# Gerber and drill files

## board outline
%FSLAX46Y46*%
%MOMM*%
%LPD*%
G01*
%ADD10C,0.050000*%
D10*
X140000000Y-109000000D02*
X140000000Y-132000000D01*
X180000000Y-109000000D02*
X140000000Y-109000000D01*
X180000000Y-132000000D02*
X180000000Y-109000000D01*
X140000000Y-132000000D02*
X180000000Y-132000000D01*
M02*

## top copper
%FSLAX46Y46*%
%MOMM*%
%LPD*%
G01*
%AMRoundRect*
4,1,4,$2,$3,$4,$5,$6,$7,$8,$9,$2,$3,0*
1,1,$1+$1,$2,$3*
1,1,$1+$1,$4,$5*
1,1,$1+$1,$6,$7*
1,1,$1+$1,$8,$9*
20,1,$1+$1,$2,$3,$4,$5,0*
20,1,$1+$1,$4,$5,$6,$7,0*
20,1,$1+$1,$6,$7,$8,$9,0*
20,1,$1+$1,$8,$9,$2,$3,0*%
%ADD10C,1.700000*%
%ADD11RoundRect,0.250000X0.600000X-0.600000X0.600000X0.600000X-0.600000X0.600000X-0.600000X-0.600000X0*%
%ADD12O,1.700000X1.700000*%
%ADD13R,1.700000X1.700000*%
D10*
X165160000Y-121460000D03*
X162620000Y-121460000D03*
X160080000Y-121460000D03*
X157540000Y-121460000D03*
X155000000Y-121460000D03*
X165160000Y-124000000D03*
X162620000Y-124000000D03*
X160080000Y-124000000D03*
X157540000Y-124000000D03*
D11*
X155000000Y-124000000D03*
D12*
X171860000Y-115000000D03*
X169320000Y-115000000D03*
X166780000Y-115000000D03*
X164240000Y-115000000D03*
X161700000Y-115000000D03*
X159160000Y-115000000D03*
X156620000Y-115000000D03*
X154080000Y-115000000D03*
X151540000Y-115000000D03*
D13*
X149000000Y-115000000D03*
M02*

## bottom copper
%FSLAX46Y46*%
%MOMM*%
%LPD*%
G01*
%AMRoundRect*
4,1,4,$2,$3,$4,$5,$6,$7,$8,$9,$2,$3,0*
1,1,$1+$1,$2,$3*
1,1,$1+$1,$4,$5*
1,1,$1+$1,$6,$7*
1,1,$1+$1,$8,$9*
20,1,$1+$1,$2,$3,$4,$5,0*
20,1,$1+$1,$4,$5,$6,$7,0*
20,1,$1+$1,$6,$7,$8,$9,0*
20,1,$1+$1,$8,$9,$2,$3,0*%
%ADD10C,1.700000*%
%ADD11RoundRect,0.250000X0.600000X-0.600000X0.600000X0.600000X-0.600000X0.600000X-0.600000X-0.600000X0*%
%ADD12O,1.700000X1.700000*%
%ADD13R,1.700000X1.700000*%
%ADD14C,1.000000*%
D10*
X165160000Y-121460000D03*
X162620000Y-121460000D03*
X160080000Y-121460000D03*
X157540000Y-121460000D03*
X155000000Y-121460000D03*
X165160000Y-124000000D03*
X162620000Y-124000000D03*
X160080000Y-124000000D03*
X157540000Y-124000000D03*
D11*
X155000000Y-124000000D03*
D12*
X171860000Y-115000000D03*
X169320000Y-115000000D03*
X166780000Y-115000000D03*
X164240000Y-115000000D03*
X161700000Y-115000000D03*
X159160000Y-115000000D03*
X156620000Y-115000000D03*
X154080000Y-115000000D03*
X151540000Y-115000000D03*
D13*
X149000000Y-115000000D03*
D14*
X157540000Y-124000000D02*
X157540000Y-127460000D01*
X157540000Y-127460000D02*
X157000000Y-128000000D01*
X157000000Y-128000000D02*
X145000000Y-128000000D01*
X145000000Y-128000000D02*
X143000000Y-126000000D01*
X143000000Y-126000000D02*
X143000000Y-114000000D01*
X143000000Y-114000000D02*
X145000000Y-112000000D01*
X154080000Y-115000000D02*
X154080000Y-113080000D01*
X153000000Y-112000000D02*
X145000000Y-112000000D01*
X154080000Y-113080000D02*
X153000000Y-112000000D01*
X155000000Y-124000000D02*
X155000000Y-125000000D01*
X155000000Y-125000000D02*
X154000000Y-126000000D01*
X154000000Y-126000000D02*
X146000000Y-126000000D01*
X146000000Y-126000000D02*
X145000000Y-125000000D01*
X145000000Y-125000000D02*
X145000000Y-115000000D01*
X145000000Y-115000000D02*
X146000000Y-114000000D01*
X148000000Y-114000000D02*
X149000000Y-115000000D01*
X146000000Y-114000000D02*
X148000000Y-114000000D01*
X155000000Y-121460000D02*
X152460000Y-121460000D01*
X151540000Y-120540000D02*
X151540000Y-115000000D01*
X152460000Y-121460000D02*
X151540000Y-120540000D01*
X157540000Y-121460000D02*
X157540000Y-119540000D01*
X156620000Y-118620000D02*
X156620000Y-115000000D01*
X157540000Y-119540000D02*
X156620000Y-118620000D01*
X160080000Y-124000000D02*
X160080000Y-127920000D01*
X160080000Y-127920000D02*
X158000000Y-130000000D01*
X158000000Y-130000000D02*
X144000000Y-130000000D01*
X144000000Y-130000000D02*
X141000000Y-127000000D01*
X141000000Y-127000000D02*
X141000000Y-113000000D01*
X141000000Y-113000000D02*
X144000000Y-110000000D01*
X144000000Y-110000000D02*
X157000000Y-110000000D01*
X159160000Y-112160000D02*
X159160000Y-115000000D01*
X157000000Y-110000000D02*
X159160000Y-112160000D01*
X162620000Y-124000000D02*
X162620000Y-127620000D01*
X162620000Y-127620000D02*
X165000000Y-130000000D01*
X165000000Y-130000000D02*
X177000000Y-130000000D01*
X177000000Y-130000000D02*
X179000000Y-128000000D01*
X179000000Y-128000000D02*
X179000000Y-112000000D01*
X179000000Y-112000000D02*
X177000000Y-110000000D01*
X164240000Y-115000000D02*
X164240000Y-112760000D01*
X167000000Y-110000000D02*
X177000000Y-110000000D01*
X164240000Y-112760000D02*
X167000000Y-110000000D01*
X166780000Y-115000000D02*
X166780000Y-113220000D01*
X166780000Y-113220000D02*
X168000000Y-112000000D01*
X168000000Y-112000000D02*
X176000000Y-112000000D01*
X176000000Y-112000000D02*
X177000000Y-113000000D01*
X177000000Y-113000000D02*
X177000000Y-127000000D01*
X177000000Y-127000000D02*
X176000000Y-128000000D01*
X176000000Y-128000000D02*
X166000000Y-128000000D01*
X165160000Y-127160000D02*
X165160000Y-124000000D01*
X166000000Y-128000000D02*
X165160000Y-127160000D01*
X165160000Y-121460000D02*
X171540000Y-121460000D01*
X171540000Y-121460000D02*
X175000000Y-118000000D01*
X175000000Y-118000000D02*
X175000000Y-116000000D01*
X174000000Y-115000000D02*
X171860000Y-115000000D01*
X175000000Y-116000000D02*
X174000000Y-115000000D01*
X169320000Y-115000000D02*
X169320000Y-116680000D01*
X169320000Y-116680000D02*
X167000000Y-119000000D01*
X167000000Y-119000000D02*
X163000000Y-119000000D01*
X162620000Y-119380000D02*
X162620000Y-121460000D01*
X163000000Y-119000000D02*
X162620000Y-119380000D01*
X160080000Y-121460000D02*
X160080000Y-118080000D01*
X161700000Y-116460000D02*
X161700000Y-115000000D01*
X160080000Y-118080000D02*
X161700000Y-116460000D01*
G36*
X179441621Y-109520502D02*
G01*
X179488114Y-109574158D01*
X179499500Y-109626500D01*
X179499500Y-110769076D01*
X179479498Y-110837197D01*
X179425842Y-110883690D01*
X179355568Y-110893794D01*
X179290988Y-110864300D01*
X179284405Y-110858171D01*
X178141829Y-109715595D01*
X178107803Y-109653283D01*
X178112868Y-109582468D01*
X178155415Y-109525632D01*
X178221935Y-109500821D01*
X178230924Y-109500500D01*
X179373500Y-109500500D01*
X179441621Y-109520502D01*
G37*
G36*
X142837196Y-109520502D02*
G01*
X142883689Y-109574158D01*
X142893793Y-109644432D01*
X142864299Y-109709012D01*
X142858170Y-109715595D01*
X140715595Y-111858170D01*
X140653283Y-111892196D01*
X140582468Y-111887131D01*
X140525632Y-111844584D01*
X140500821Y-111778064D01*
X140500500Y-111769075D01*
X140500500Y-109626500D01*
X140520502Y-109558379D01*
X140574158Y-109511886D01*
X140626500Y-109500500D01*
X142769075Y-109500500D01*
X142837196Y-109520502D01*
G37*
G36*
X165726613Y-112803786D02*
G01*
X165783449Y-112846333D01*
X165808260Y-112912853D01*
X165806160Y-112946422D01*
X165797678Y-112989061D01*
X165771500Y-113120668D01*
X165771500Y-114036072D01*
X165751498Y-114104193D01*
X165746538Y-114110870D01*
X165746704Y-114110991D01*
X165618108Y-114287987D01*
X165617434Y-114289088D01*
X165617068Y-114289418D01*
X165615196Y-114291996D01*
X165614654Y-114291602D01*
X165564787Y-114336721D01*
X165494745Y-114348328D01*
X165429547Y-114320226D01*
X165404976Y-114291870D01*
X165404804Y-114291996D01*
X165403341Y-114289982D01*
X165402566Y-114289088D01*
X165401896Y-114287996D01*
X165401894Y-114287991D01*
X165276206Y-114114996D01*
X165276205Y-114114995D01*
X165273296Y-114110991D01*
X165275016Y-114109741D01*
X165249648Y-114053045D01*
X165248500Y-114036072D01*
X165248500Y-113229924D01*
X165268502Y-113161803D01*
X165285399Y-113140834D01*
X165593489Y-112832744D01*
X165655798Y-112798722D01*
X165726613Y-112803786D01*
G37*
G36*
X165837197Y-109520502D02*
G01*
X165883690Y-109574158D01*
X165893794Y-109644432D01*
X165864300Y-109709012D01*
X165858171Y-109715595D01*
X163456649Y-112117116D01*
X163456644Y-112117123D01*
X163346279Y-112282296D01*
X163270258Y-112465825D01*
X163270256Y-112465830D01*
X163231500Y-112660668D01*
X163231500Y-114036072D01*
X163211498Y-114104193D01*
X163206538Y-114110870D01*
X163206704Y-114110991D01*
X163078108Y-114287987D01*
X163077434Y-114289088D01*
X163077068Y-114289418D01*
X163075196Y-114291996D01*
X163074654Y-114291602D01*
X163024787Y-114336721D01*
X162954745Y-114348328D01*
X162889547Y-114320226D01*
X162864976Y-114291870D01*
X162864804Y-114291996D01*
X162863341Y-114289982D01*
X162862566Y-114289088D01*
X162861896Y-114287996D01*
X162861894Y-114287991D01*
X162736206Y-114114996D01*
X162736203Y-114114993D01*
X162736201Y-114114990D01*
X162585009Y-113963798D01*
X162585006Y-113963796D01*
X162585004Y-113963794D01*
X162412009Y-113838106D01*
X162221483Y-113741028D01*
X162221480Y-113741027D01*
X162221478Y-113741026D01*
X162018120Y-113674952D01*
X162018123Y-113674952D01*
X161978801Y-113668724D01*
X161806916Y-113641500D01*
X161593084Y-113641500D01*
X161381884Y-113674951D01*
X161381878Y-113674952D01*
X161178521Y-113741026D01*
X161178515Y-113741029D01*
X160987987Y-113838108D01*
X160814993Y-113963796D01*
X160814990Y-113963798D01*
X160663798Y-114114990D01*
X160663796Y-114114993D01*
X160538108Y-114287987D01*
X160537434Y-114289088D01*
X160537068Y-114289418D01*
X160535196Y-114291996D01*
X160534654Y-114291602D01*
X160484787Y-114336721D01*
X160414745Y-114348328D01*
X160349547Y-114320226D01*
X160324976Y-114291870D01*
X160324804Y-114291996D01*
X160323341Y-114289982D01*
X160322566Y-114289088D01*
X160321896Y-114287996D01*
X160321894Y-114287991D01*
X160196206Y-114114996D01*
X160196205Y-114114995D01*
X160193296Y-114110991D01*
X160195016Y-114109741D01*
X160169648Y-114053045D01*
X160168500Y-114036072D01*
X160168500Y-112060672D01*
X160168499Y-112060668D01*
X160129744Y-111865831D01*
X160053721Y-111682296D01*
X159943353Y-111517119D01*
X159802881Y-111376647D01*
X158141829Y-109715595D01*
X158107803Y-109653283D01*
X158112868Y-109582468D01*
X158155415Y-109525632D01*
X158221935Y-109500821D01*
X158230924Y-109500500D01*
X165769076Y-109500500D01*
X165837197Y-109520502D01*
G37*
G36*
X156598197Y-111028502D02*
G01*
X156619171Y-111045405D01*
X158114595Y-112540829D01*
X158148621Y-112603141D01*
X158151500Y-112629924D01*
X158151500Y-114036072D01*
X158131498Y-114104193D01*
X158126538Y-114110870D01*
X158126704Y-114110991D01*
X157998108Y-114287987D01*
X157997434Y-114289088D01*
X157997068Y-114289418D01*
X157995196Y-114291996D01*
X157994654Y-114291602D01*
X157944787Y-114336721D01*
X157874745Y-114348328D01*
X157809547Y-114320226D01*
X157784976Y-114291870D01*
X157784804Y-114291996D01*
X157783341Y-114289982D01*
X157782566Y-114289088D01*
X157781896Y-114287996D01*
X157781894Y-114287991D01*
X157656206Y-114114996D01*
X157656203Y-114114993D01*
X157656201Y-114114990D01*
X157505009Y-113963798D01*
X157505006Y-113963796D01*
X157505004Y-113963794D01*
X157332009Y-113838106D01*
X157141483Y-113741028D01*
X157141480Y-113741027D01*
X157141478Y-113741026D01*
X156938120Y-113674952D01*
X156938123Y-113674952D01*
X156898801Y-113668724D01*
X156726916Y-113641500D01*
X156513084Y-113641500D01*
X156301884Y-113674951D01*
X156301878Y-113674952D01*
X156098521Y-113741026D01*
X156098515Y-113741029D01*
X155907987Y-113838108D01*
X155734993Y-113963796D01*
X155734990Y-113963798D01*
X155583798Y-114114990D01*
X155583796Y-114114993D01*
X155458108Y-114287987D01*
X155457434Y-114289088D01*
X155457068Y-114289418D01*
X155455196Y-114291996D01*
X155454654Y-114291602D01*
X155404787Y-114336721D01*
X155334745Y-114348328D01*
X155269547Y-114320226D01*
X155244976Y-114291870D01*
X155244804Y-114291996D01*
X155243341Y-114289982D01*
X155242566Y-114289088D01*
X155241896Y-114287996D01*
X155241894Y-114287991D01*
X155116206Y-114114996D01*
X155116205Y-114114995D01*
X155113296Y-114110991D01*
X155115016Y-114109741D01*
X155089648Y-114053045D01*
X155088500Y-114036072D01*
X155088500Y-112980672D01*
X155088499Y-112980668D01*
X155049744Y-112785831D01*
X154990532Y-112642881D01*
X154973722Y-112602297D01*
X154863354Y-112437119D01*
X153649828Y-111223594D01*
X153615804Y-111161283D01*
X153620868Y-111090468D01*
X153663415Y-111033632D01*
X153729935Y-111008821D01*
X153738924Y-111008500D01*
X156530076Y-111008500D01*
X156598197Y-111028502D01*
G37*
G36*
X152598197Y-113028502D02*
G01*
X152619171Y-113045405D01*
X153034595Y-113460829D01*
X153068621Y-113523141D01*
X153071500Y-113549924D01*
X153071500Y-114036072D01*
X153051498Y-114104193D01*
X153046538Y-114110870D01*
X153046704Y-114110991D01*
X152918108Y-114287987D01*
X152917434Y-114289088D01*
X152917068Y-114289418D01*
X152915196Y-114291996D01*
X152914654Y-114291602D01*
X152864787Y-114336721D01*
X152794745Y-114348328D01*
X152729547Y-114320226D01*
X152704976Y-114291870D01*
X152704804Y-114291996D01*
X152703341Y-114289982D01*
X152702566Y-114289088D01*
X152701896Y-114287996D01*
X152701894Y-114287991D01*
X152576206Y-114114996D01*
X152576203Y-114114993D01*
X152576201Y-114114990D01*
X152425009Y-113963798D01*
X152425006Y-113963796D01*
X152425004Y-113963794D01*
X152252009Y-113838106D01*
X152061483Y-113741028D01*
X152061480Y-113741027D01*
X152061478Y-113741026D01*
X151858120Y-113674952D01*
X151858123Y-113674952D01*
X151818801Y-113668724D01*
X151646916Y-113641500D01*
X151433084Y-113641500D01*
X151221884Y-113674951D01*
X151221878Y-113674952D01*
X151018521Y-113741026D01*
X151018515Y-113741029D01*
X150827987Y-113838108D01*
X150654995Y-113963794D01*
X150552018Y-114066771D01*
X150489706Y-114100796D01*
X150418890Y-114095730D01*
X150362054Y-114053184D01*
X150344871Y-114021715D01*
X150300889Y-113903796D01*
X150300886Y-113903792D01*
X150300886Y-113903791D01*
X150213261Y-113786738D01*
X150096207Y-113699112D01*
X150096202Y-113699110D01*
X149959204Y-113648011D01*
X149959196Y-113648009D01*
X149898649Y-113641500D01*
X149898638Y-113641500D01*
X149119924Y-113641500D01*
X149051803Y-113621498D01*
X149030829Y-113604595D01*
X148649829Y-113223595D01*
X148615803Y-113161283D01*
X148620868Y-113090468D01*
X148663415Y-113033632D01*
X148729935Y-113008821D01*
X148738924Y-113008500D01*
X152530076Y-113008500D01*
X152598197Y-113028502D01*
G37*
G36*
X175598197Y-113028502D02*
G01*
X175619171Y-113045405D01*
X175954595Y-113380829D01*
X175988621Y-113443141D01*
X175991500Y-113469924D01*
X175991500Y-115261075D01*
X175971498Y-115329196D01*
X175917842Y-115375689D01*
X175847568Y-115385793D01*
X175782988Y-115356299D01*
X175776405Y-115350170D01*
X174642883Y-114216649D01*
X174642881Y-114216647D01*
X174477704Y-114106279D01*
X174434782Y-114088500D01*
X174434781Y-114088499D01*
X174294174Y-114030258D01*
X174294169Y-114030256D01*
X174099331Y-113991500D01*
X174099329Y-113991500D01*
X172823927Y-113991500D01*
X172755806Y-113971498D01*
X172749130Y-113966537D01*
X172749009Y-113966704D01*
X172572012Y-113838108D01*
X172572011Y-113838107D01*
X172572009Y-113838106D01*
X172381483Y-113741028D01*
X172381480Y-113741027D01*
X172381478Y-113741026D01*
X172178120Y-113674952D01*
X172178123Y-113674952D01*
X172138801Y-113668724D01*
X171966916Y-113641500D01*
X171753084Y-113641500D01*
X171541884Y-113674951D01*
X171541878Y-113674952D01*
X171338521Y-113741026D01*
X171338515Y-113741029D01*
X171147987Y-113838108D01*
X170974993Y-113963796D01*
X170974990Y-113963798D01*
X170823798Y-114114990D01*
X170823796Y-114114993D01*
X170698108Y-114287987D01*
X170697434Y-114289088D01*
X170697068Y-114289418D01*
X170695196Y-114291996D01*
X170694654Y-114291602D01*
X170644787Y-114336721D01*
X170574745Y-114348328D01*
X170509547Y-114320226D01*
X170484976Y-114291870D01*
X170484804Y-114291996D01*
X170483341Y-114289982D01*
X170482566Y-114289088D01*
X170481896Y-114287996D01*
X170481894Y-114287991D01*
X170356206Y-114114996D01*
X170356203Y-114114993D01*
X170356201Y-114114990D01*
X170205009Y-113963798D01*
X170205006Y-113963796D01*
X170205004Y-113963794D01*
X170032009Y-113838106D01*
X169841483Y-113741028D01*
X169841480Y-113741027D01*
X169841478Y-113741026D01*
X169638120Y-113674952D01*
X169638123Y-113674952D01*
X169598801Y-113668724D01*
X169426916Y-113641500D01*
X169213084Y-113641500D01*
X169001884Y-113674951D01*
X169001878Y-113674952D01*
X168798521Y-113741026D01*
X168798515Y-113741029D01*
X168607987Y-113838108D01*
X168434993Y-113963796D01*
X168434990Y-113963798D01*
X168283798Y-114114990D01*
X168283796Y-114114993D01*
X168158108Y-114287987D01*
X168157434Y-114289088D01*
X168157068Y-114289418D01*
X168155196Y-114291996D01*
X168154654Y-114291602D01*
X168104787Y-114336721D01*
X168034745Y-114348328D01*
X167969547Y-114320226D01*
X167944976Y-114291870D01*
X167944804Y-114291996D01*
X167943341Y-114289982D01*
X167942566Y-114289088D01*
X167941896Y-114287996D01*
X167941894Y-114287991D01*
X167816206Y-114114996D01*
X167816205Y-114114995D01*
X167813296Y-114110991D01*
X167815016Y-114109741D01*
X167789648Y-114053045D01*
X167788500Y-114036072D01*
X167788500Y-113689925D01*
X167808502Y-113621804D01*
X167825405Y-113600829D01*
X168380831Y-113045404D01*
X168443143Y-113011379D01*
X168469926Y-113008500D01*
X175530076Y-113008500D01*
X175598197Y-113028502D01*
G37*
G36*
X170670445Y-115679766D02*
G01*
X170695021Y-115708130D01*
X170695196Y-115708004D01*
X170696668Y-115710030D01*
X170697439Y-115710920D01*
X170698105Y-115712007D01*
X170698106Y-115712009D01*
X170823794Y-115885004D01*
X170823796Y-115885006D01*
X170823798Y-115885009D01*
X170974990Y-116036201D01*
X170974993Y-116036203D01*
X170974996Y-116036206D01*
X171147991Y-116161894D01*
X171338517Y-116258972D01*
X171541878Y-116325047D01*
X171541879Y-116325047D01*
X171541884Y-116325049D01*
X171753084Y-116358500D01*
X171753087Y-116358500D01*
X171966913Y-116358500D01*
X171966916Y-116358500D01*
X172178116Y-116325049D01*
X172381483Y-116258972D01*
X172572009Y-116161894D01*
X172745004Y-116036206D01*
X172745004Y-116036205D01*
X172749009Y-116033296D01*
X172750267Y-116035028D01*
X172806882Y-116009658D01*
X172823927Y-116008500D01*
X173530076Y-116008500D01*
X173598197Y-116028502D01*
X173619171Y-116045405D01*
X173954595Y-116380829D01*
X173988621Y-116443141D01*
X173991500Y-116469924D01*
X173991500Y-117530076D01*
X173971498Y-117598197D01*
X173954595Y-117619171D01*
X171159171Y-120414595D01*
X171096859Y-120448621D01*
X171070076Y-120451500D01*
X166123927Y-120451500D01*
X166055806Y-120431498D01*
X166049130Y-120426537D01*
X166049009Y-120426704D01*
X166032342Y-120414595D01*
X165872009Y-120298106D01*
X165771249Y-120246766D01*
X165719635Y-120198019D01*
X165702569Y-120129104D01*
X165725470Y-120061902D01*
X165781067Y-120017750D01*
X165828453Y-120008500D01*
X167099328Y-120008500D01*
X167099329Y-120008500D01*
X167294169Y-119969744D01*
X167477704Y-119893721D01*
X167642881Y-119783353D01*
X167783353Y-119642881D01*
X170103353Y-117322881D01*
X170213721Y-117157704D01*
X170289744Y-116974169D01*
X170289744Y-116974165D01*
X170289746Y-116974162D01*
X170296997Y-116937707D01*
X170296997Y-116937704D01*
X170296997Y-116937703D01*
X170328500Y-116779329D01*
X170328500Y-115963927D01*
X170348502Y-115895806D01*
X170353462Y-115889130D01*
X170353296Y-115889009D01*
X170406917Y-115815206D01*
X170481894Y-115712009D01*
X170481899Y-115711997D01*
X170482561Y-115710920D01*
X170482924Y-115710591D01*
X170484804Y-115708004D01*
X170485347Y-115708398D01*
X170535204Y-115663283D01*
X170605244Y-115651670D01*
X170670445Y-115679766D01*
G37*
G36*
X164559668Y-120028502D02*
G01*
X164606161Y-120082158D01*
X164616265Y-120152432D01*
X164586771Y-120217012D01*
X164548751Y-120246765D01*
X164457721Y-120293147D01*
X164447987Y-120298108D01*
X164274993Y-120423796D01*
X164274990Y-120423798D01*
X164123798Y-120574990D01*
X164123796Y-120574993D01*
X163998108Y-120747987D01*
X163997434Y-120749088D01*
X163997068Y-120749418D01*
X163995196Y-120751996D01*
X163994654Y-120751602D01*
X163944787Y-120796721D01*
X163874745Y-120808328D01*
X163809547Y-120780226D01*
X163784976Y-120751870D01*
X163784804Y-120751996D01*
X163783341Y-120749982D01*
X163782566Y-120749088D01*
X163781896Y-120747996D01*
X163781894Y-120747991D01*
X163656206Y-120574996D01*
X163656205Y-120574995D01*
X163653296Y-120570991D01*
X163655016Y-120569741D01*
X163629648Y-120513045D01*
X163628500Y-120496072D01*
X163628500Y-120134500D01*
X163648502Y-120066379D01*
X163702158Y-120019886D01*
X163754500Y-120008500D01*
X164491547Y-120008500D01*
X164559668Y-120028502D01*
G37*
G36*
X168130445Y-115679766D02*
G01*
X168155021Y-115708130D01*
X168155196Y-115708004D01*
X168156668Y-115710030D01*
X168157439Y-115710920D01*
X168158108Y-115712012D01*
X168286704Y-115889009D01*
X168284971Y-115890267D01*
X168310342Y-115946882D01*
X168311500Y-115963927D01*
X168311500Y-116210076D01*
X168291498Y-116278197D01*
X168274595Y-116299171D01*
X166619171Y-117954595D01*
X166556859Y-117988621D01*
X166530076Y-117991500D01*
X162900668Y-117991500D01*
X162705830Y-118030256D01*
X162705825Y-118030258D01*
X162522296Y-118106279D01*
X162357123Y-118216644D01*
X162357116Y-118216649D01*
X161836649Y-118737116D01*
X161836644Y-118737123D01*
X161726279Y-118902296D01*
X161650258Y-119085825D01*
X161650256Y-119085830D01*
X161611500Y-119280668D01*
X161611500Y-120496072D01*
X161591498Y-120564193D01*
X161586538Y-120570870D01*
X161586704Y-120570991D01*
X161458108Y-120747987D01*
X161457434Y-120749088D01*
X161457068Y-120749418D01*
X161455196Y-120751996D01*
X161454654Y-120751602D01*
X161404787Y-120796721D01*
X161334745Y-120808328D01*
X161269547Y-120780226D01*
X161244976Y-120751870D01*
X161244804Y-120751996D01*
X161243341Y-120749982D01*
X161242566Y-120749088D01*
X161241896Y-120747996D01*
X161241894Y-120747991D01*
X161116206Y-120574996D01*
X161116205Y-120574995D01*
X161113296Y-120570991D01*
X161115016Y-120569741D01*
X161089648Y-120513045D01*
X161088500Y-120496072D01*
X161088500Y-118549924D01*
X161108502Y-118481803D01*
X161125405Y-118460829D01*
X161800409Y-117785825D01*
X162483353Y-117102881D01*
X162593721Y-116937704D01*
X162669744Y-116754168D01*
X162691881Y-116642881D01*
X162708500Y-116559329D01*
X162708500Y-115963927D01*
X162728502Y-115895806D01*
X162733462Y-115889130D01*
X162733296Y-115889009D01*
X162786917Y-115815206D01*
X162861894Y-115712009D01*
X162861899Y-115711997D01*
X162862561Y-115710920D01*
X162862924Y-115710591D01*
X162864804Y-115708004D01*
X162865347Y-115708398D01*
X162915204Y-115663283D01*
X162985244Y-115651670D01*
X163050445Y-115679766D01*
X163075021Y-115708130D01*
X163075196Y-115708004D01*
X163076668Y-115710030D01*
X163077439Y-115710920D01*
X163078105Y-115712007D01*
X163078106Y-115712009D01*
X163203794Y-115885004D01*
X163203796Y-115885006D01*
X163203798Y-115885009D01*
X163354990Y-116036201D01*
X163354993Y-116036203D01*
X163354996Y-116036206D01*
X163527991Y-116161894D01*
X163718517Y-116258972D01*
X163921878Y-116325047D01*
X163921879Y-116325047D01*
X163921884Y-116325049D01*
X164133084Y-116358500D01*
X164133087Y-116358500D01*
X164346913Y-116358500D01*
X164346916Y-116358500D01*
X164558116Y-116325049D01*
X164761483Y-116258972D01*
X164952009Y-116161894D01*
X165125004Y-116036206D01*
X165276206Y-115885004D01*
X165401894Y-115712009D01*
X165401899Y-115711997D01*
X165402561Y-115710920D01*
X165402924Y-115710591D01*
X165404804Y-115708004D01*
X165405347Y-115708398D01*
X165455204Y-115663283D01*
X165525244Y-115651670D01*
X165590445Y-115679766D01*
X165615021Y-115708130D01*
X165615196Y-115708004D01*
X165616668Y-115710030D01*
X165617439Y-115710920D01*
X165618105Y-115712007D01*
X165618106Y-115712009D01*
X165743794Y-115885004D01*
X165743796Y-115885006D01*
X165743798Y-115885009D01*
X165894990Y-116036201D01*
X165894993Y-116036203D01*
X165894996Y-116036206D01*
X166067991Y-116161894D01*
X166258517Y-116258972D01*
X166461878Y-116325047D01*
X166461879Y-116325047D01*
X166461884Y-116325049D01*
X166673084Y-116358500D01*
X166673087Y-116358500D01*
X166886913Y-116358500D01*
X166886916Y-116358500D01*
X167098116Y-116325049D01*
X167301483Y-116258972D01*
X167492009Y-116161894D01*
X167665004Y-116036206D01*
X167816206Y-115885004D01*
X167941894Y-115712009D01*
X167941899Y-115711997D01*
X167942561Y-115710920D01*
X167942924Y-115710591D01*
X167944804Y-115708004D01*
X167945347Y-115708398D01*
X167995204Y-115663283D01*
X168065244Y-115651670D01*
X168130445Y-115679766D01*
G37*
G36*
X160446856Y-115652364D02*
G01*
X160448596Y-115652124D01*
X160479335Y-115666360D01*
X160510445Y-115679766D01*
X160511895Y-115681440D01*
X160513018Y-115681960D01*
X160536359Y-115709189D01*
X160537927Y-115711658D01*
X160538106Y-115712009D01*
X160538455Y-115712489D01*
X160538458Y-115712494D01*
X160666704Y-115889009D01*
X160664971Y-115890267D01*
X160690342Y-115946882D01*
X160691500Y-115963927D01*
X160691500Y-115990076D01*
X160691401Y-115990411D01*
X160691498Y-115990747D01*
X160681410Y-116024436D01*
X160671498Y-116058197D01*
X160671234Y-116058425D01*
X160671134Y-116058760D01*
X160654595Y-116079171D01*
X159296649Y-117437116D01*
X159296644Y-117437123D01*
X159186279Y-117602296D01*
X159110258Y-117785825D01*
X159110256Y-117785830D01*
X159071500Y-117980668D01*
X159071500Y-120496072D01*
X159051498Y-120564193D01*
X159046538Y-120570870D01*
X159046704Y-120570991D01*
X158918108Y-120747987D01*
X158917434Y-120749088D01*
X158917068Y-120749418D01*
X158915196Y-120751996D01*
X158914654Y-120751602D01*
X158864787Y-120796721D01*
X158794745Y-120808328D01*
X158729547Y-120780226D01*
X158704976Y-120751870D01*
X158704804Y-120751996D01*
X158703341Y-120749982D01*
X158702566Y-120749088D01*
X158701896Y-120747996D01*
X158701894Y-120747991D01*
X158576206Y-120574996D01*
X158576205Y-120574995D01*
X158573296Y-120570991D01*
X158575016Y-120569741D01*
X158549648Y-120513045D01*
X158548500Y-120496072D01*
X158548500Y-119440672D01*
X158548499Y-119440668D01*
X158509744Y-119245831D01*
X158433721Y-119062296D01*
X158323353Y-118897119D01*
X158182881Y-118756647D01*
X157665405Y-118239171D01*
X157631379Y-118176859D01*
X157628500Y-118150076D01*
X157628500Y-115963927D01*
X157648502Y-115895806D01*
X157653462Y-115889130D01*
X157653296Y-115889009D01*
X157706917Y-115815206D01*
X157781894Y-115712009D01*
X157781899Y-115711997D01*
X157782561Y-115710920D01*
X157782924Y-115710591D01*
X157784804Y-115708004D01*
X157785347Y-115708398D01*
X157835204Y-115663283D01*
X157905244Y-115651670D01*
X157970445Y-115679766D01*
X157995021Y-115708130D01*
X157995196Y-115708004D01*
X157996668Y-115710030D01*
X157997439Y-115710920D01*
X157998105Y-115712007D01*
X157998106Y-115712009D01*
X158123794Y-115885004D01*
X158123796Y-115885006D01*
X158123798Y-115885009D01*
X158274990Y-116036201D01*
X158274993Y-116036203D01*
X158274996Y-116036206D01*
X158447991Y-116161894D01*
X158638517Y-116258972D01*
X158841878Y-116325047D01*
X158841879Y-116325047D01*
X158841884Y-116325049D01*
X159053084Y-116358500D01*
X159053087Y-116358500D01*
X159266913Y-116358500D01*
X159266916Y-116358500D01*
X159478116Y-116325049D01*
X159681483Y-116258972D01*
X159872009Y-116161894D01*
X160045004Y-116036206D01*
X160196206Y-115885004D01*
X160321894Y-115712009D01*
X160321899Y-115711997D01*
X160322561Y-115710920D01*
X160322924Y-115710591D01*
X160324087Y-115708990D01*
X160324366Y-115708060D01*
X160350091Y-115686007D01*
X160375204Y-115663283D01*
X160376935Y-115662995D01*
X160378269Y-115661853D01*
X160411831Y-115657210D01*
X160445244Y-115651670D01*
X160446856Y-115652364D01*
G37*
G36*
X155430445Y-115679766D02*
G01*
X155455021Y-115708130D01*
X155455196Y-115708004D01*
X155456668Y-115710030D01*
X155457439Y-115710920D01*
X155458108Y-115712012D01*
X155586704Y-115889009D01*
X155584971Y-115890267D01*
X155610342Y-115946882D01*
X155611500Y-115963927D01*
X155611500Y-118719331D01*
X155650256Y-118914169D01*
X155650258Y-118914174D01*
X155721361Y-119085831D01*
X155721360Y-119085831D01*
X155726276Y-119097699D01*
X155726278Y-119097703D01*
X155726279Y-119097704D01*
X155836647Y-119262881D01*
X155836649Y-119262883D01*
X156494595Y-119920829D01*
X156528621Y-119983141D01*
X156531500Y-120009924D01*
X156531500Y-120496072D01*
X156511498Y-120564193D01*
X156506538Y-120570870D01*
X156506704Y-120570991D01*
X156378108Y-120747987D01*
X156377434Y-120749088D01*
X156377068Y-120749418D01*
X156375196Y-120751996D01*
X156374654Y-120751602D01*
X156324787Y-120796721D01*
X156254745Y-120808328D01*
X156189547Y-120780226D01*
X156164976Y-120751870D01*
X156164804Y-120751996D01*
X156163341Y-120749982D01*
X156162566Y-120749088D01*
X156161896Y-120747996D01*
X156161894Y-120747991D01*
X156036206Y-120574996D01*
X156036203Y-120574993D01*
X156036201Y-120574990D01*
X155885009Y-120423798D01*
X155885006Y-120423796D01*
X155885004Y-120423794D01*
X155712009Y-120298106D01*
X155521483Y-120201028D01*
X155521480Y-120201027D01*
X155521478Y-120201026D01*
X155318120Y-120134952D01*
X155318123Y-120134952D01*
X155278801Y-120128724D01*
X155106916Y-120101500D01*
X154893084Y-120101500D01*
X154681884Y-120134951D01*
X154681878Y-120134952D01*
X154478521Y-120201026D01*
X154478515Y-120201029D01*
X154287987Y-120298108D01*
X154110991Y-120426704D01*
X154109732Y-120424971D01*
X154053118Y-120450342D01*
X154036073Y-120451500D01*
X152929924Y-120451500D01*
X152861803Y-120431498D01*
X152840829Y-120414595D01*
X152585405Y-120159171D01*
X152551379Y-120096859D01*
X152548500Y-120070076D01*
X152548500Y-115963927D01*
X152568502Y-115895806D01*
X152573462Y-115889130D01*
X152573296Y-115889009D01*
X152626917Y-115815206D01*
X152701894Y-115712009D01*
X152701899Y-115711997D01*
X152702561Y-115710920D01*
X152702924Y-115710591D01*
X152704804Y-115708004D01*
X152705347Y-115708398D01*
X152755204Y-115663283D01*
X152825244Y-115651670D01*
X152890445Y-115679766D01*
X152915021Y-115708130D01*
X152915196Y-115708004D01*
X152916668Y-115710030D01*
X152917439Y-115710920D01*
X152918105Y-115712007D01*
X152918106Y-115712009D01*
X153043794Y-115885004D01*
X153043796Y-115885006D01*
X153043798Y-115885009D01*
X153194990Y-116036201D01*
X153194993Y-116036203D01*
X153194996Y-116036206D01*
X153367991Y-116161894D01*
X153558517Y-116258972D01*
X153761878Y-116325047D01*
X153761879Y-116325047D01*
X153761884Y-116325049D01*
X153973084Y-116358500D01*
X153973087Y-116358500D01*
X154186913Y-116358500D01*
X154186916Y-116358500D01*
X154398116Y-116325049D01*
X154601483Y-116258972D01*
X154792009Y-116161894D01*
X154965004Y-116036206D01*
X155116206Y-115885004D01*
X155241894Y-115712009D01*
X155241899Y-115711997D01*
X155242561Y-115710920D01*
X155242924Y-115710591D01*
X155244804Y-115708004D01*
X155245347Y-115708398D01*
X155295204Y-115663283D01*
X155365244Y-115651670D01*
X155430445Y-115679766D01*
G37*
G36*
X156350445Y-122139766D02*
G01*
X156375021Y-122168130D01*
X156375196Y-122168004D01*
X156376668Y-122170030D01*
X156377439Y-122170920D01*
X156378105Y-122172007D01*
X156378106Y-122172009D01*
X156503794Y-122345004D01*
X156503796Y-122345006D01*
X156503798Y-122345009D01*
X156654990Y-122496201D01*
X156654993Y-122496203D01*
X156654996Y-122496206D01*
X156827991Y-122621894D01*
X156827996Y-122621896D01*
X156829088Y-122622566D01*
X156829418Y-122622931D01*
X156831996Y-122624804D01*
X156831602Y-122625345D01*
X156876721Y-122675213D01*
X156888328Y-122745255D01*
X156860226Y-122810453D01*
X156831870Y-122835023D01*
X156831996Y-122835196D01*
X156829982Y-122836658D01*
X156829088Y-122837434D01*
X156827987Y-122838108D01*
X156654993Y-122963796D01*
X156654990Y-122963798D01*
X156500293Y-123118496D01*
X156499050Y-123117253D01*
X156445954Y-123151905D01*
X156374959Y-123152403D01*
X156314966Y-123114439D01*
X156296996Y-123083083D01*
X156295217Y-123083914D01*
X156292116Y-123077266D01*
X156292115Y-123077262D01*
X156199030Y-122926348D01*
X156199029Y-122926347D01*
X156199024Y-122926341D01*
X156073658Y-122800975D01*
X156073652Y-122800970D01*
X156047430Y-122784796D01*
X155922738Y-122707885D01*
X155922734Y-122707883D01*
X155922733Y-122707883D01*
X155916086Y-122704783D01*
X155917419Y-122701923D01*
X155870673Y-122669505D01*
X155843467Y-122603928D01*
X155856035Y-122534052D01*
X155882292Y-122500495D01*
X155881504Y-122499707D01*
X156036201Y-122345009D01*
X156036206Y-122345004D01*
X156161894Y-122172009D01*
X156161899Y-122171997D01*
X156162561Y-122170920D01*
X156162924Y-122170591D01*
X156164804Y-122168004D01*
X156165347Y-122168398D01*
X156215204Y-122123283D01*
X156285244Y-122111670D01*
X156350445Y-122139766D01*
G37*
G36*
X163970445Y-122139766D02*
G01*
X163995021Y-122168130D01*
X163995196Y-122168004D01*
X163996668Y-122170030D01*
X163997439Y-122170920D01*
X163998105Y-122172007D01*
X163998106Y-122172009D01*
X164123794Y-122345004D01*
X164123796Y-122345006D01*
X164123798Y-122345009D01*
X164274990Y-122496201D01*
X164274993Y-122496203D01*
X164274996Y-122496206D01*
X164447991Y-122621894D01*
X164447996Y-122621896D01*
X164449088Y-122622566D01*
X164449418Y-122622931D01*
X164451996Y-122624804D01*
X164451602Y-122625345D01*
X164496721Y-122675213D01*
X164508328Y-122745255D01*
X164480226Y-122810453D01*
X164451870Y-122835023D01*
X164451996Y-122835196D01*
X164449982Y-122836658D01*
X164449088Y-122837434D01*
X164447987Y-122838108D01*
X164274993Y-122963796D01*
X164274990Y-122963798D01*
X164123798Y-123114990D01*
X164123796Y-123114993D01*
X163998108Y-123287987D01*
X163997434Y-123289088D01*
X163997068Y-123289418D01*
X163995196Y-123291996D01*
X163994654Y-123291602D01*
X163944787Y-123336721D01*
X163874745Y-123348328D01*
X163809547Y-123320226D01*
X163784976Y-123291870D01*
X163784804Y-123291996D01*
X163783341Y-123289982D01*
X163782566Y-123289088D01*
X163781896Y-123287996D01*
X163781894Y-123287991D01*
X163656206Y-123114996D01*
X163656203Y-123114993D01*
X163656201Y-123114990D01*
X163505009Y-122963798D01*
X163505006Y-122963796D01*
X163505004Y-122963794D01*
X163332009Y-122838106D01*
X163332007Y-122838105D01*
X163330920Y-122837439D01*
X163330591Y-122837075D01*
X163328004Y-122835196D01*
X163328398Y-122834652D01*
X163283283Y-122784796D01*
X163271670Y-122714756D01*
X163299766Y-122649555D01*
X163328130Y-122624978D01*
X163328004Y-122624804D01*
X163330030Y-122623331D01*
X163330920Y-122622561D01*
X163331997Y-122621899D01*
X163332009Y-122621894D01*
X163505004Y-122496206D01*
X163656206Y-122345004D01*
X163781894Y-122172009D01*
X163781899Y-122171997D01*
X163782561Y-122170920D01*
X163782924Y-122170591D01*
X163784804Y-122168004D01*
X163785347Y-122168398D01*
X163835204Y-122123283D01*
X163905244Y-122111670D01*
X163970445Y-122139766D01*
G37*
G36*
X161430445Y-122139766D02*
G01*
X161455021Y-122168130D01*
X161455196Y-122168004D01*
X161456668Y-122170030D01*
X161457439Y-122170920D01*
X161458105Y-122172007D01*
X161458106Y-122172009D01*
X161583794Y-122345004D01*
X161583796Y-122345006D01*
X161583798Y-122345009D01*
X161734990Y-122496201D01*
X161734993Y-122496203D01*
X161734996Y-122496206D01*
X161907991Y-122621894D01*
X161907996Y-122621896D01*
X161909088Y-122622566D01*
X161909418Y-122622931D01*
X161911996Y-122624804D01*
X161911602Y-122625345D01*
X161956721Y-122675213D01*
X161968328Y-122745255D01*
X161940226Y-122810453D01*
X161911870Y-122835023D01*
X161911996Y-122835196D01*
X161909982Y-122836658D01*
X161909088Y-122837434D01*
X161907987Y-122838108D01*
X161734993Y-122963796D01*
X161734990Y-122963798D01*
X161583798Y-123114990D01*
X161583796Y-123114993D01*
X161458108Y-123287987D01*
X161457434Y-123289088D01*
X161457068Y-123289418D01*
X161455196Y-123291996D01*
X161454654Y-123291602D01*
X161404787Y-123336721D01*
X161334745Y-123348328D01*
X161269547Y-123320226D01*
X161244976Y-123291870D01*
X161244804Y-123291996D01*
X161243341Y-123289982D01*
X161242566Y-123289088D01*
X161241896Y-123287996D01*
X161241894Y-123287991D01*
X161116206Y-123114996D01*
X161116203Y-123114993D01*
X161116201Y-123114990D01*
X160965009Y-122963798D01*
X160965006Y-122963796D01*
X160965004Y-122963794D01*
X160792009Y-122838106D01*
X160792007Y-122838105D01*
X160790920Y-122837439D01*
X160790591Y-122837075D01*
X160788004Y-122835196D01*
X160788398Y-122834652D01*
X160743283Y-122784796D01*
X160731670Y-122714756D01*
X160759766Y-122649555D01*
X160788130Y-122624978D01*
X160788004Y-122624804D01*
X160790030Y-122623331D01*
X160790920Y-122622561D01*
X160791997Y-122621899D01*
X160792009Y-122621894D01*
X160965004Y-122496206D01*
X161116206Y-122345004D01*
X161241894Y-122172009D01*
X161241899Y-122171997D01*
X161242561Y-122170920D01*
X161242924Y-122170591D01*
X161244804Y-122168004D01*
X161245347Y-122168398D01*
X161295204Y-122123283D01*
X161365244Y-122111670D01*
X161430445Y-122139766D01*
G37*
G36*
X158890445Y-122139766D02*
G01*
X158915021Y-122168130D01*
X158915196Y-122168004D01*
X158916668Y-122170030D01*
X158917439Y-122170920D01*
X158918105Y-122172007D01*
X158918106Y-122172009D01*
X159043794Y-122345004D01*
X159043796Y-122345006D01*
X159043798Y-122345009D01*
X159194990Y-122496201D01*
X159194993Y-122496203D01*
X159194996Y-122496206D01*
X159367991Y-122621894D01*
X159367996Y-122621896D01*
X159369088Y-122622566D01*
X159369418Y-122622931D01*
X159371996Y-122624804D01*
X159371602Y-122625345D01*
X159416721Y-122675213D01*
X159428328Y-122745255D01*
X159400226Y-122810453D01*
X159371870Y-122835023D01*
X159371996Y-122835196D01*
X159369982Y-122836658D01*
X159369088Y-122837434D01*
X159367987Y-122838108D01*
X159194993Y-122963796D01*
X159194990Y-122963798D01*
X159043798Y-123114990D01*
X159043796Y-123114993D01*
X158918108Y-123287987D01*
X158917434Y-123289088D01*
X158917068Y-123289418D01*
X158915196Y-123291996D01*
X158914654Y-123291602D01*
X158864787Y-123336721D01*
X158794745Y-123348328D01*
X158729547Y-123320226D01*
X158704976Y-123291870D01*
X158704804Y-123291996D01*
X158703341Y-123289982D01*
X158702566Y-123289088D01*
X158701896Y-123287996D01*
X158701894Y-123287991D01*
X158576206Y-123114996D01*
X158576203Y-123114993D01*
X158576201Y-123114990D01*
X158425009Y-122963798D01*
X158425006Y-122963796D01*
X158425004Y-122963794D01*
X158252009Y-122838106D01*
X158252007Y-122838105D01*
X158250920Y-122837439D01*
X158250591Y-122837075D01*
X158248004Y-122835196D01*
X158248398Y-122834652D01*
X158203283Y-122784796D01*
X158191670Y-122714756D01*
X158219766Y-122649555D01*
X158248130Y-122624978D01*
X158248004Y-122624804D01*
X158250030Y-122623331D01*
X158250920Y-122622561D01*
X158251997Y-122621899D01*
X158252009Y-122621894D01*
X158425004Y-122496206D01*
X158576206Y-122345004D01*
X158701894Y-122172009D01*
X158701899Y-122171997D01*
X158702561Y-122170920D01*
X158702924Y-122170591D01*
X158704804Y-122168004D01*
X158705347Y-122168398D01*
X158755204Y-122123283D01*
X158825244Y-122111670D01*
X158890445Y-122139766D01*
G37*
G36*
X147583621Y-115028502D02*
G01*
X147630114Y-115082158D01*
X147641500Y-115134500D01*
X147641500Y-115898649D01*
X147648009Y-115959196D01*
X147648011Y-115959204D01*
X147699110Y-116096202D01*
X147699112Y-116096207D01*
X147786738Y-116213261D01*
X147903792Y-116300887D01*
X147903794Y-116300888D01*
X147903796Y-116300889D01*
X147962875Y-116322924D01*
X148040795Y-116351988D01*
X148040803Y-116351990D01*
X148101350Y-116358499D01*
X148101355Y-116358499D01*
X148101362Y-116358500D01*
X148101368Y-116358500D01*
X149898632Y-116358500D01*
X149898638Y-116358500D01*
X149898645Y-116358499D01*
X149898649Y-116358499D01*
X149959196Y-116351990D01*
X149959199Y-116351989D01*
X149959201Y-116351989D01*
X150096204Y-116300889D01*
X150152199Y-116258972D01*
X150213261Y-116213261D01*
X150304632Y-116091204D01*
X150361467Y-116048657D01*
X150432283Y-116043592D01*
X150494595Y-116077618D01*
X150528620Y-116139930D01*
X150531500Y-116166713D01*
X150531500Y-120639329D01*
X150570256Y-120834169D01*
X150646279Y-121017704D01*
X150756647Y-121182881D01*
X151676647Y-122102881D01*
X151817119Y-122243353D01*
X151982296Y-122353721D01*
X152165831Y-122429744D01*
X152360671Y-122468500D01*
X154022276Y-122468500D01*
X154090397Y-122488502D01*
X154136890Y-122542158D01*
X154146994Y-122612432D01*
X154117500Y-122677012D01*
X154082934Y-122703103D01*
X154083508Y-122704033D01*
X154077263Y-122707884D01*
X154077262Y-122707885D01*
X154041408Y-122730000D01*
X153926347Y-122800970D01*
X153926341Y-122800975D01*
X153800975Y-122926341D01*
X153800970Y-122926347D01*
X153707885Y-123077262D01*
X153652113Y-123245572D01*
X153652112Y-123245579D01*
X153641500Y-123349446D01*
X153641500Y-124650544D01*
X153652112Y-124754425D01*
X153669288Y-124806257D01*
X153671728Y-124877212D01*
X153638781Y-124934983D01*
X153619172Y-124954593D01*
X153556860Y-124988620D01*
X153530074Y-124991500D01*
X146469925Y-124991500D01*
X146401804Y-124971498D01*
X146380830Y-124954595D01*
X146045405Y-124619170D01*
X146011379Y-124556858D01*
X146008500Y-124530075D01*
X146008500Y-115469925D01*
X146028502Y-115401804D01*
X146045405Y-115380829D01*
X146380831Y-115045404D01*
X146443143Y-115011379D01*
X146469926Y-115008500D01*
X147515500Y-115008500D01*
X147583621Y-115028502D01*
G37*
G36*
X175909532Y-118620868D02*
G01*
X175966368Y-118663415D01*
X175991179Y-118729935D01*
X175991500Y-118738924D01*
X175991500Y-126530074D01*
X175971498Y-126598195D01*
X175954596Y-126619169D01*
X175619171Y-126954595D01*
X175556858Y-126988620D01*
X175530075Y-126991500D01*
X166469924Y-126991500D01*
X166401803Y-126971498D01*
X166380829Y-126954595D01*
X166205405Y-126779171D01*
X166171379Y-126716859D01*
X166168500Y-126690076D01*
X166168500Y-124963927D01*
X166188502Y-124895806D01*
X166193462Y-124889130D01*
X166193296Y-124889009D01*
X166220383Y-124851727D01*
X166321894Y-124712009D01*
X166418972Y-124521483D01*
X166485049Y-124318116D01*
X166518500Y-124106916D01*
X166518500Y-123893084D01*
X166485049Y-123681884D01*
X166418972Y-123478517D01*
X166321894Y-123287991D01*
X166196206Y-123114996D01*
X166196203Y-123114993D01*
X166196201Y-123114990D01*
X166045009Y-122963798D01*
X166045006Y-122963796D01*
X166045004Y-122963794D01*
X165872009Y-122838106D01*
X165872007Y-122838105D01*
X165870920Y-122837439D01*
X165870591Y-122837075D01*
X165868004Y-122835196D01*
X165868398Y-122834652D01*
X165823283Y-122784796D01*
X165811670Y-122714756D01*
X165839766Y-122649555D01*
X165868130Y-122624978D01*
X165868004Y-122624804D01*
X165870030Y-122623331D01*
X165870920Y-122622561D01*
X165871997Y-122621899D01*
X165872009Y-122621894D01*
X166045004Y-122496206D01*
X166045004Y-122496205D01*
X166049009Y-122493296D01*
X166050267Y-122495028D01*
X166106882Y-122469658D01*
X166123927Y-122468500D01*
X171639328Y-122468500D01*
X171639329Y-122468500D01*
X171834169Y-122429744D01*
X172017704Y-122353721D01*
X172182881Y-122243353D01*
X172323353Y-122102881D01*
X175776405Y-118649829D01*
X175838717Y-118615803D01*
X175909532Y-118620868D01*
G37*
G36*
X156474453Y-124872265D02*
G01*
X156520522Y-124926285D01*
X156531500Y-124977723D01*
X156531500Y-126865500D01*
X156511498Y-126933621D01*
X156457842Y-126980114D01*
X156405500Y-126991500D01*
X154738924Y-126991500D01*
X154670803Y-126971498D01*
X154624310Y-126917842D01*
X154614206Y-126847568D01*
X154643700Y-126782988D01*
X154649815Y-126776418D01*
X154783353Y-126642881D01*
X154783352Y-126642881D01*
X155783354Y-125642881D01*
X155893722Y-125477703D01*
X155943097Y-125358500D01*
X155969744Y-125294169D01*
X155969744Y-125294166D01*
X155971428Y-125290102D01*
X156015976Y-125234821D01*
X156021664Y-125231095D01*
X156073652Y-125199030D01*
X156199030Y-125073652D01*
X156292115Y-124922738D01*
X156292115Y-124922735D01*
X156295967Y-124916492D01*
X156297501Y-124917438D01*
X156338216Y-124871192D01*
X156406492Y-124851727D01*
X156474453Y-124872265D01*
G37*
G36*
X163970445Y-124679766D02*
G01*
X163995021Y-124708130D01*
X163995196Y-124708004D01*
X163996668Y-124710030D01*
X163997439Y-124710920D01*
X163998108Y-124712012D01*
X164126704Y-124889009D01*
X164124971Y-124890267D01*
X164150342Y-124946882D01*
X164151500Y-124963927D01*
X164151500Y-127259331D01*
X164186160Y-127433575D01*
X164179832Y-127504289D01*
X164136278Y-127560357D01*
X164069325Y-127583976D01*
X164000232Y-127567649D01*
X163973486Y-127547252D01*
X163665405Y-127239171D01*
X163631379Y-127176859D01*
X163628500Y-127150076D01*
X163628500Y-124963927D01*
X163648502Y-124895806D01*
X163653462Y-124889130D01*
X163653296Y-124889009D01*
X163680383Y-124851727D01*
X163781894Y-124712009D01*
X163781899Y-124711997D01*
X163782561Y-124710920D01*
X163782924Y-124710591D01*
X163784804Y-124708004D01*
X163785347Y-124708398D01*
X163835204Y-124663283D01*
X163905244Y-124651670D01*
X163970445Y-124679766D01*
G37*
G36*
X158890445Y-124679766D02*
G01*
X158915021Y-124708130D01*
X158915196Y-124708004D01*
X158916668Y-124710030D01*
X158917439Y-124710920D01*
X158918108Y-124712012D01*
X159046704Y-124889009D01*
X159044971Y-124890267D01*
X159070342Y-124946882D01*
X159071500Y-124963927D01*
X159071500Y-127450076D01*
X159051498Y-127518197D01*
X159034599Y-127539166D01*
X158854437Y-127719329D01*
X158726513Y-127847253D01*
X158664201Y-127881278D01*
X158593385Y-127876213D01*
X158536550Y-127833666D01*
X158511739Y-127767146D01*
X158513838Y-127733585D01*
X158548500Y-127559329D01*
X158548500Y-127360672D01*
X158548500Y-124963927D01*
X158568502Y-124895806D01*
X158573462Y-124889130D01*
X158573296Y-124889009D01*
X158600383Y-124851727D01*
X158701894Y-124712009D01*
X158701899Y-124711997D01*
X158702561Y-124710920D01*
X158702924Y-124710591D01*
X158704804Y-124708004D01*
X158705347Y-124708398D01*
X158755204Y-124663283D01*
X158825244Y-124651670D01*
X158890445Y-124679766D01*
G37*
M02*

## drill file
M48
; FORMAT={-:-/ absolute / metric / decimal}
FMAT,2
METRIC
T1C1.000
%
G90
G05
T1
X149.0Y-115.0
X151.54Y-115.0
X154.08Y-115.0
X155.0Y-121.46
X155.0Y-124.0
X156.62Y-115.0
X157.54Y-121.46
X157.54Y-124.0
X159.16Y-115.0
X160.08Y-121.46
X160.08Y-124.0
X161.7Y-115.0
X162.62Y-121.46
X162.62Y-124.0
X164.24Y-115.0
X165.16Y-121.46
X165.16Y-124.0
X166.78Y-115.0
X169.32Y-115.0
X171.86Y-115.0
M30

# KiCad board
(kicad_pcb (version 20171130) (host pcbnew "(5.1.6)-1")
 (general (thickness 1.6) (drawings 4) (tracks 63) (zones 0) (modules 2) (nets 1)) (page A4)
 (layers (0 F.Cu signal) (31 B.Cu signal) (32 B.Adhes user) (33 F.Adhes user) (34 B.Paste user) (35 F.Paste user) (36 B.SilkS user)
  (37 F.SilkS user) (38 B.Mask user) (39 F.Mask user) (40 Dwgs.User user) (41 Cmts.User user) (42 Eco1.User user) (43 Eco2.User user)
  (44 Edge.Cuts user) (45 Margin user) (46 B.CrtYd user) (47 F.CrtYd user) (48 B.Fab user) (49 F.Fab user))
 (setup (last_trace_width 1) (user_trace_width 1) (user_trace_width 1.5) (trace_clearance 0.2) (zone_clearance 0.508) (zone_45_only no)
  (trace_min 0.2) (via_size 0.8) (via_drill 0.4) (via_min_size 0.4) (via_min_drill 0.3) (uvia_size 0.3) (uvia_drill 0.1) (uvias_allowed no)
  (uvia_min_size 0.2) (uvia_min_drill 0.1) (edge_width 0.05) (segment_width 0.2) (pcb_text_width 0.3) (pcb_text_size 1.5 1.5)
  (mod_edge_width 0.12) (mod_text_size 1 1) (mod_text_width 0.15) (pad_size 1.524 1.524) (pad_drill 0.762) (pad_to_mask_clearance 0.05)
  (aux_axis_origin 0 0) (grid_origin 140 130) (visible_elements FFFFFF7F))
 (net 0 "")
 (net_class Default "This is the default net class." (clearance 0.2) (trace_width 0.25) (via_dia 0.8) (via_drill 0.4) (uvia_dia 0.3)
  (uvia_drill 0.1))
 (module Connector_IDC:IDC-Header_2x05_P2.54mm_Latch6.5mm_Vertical (layer F.Cu) (at 155 124 90)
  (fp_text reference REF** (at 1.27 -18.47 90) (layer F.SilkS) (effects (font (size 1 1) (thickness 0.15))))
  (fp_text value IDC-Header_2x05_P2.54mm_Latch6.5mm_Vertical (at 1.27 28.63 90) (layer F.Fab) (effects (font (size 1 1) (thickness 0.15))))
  (pad 10 thru_hole circle (at 2.54 10.16 90) (size 1.7 1.7) (drill 1) (layers *.Cu *.Mask))
  (pad 8 thru_hole circle (at 2.54 7.62 90) (size 1.7 1.7) (drill 1) (layers *.Cu *.Mask))
  (pad 6 thru_hole circle (at 2.54 5.08 90) (size 1.7 1.7) (drill 1) (layers *.Cu *.Mask))
  (pad 4 thru_hole circle (at 2.54 2.54 90) (size 1.7 1.7) (drill 1) (layers *.Cu *.Mask))
  (pad 2 thru_hole circle (at 2.54 0 90) (size 1.7 1.7) (drill 1) (layers *.Cu *.Mask))
  (pad 9 thru_hole circle (at 0 10.16 90) (size 1.7 1.7) (drill 1) (layers *.Cu *.Mask))
  (pad 7 thru_hole circle (at 0 7.62 90) (size 1.7 1.7) (drill 1) (layers *.Cu *.Mask))
  (pad 5 thru_hole circle (at 0 5.08 90) (size 1.7 1.7) (drill 1) (layers *.Cu *.Mask))
  (pad 3 thru_hole circle (at 0 2.54 90) (size 1.7 1.7) (drill 1) (layers *.Cu *.Mask))
  (pad 1 thru_hole roundrect (at 0 0 90) (size 1.7 1.7) (drill 1) (layers *.Cu *.Mask) (roundrect_rratio 0.147059)))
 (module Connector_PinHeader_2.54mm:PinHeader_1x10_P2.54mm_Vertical (layer F.Cu) (at 149 115 90)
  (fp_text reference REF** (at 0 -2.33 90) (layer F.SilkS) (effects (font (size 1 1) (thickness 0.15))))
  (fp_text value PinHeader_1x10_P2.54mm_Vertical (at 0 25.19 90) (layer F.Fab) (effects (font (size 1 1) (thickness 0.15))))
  (pad 10 thru_hole oval (at 0 22.86 90) (size 1.7 1.7) (drill 1) (layers *.Cu *.Mask))
  (pad 9 thru_hole oval (at 0 20.32 90) (size 1.7 1.7) (drill 1) (layers *.Cu *.Mask))
  (pad 8 thru_hole oval (at 0 17.78 90) (size 1.7 1.7) (drill 1) (layers *.Cu *.Mask))
  (pad 7 thru_hole oval (at 0 15.24 90) (size 1.7 1.7) (drill 1) (layers *.Cu *.Mask))
  (pad 6 thru_hole oval (at 0 12.7 90) (size 1.7 1.7) (drill 1) (layers *.Cu *.Mask))
  (pad 5 thru_hole oval (at 0 10.16 90) (size 1.7 1.7) (drill 1) (layers *.Cu *.Mask))
  (pad 4 thru_hole oval (at 0 7.62 90) (size 1.7 1.7) (drill 1) (layers *.Cu *.Mask))
  (pad 3 thru_hole oval (at 0 5.08 90) (size 1.7 1.7) (drill 1) (layers *.Cu *.Mask))
  (pad 2 thru_hole oval (at 0 2.54 90) (size 1.7 1.7) (drill 1) (layers *.Cu *.Mask))
  (pad 1 thru_hole rect (at 0 0 90) (size 1.7 1.7) (drill 1) (layers *.Cu *.Mask)))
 (gr_line (start 140 109) (end 140 132) (layer Edge.Cuts) (width 0.05))
 (gr_line (start 180 109) (end 140 109) (layer Edge.Cuts) (width 0.05))
 (gr_line (start 180 132) (end 180 109) (layer Edge.Cuts) (width 0.05))
 (gr_line (start 140 132) (end 180 132) (layer Edge.Cuts) (width 0.05))
 (segment (start 157.54 124) (end 157.54 127.46) (width 1) (layer B.Cu) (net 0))
 (segment (start 157.54 127.46) (end 157 128) (width 1) (layer B.Cu) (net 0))
 (segment (start 157 128) (end 145 128) (width 1) (layer B.Cu) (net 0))
 (segment (start 145 128) (end 143 126) (width 1) (layer B.Cu) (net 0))
 (segment (start 143 126) (end 143 114) (width 1) (layer B.Cu) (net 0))
 (segment (start 143 114) (end 145 112) (width 1) (layer B.Cu) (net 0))
 (segment (start 154.08 115) (end 154.08 113.08) (width 1) (layer B.Cu) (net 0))
 (segment (start 153 112) (end 145 112) (width 1) (layer B.Cu) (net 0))
 (segment (start 154.08 113.08) (end 153 112) (width 1) (layer B.Cu) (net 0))
 (segment (start 155 124) (end 155 125) (width 1) (layer B.Cu) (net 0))
 (segment (start 155 125) (end 154 126) (width 1) (layer B.Cu) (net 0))
 (segment (start 154 126) (end 146 126) (width 1) (layer B.Cu) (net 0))
 (segment (start 146 126) (end 145 125) (width 1) (layer B.Cu) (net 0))
 (segment (start 145 125) (end 145 115) (width 1) (layer B.Cu) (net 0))
 (segment (start 145 115) (end 146 114) (width 1) (layer B.Cu) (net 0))
 (segment (start 148 114) (end 149 115) (width 1) (layer B.Cu) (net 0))
 (segment (start 146 114) (end 148 114) (width 1) (layer B.Cu) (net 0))
 (segment (start 155 121.46) (end 152.46 121.46) (width 1) (layer B.Cu) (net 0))
 (segment (start 151.54 120.54) (end 151.54 115) (width 1) (layer B.Cu) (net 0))
 (segment (start 152.46 121.46) (end 151.54 120.54) (width 1) (layer B.Cu) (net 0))
 (segment (start 157.54 121.46) (end 157.54 119.54) (width 1) (layer B.Cu) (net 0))
 (segment (start 156.62 118.62) (end 156.62 115) (width 1) (layer B.Cu) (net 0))
 (segment (start 157.54 119.54) (end 156.62 118.62) (width 1) (layer B.Cu) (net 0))
 (segment (start 160.08 124) (end 160.08 127.92) (width 1) (layer B.Cu) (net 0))
 (segment (start 160.08 127.92) (end 158 130) (width 1) (layer B.Cu) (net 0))
 (segment (start 158 130) (end 144 130) (width 1) (layer B.Cu) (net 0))
 (segment (start 144 130) (end 141 127) (width 1) (layer B.Cu) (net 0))
 (segment (start 141 127) (end 141 113) (width 1) (layer B.Cu) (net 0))
 (segment (start 141 113) (end 144 110) (width 1) (layer B.Cu) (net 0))
 (segment (start 144 110) (end 157 110) (width 1) (layer B.Cu) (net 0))
 (segment (start 159.16 112.16) (end 159.16 115) (width 1) (layer B.Cu) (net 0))
 (segment (start 157 110) (end 159.16 112.16) (width 1) (layer B.Cu) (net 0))
 (segment (start 162.62 124) (end 162.62 127.62) (width 1) (layer B.Cu) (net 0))
 (segment (start 162.62 127.62) (end 165 130) (width 1) (layer B.Cu) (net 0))
 (segment (start 165 130) (end 177 130) (width 1) (layer B.Cu) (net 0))
 (segment (start 177 130) (end 179 128) (width 1) (layer B.Cu) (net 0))
 (segment (start 179 128) (end 179 112) (width 1) (layer B.Cu) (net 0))
 (segment (start 179 112) (end 177 110) (width 1) (layer B.Cu) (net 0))
 (segment (start 164.24 115) (end 164.24 112.76) (width 1) (layer B.Cu) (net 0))
 (segment (start 167 110) (end 177 110) (width 1) (layer B.Cu) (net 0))
 (segment (start 164.24 112.76) (end 167 110) (width 1) (layer B.Cu) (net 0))
 (segment (start 166.78 115) (end 166.78 113.22) (width 1) (layer B.Cu) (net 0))
 (segment (start 166.78 113.22) (end 168 112) (width 1) (layer B.Cu) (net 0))
 (segment (start 168 112) (end 176 112) (width 1) (layer B.Cu) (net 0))
 (segment (start 176 112) (end 177 113) (width 1) (layer B.Cu) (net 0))
 (segment (start 177 113) (end 177 127) (width 1) (layer B.Cu) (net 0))
 (segment (start 177 127) (end 176 128) (width 1) (layer B.Cu) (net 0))
 (segment (start 176 128) (end 166 128) (width 1) (layer B.Cu) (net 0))
 (segment (start 165.16 127.16) (end 165.16 124) (width 1) (layer B.Cu) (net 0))
 (segment (start 166 128) (end 165.16 127.16) (width 1) (layer B.Cu) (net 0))
 (segment (start 165.16 121.46) (end 171.54 121.46) (width 1) (layer B.Cu) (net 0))
 (segment (start 171.54 121.46) (end 175 118) (width 1) (layer B.Cu) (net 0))
 (segment (start 175 118) (end 175 116) (width 1) (layer B.Cu) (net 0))
 (segment (start 174 115) (end 171.86 115) (width 1) (layer B.Cu) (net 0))
 (segment (start 175 116) (end 174 115) (width 1) (layer B.Cu) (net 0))
 (segment (start 169.32 115) (end 169.32 116.68) (width 1) (layer B.Cu) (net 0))
 (segment (start 169.32 116.68) (end 167 119) (width 1) (layer B.Cu) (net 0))
 (segment (start 167 119) (end 163 119) (width 1) (layer B.Cu) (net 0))
 (segment (start 162.62 119.38) (end 162.62 121.46) (width 1) (layer B.Cu) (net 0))
 (segment (start 163 119) (end 162.62 119.38) (width 1) (layer B.Cu) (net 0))
 (segment (start 160.08 121.46) (end 160.08 118.08) (width 1) (layer B.Cu) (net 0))
 (segment (start 161.7 116.46) (end 161.7 115) (width 1) (layer B.Cu) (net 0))
 (segment (start 160.08 118.08) (end 161.7 116.46) (width 1) (layer B.Cu) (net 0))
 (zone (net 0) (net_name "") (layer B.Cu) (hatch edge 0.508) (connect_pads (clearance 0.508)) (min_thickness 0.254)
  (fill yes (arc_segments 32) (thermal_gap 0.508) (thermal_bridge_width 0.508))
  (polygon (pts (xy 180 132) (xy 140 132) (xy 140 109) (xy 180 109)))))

